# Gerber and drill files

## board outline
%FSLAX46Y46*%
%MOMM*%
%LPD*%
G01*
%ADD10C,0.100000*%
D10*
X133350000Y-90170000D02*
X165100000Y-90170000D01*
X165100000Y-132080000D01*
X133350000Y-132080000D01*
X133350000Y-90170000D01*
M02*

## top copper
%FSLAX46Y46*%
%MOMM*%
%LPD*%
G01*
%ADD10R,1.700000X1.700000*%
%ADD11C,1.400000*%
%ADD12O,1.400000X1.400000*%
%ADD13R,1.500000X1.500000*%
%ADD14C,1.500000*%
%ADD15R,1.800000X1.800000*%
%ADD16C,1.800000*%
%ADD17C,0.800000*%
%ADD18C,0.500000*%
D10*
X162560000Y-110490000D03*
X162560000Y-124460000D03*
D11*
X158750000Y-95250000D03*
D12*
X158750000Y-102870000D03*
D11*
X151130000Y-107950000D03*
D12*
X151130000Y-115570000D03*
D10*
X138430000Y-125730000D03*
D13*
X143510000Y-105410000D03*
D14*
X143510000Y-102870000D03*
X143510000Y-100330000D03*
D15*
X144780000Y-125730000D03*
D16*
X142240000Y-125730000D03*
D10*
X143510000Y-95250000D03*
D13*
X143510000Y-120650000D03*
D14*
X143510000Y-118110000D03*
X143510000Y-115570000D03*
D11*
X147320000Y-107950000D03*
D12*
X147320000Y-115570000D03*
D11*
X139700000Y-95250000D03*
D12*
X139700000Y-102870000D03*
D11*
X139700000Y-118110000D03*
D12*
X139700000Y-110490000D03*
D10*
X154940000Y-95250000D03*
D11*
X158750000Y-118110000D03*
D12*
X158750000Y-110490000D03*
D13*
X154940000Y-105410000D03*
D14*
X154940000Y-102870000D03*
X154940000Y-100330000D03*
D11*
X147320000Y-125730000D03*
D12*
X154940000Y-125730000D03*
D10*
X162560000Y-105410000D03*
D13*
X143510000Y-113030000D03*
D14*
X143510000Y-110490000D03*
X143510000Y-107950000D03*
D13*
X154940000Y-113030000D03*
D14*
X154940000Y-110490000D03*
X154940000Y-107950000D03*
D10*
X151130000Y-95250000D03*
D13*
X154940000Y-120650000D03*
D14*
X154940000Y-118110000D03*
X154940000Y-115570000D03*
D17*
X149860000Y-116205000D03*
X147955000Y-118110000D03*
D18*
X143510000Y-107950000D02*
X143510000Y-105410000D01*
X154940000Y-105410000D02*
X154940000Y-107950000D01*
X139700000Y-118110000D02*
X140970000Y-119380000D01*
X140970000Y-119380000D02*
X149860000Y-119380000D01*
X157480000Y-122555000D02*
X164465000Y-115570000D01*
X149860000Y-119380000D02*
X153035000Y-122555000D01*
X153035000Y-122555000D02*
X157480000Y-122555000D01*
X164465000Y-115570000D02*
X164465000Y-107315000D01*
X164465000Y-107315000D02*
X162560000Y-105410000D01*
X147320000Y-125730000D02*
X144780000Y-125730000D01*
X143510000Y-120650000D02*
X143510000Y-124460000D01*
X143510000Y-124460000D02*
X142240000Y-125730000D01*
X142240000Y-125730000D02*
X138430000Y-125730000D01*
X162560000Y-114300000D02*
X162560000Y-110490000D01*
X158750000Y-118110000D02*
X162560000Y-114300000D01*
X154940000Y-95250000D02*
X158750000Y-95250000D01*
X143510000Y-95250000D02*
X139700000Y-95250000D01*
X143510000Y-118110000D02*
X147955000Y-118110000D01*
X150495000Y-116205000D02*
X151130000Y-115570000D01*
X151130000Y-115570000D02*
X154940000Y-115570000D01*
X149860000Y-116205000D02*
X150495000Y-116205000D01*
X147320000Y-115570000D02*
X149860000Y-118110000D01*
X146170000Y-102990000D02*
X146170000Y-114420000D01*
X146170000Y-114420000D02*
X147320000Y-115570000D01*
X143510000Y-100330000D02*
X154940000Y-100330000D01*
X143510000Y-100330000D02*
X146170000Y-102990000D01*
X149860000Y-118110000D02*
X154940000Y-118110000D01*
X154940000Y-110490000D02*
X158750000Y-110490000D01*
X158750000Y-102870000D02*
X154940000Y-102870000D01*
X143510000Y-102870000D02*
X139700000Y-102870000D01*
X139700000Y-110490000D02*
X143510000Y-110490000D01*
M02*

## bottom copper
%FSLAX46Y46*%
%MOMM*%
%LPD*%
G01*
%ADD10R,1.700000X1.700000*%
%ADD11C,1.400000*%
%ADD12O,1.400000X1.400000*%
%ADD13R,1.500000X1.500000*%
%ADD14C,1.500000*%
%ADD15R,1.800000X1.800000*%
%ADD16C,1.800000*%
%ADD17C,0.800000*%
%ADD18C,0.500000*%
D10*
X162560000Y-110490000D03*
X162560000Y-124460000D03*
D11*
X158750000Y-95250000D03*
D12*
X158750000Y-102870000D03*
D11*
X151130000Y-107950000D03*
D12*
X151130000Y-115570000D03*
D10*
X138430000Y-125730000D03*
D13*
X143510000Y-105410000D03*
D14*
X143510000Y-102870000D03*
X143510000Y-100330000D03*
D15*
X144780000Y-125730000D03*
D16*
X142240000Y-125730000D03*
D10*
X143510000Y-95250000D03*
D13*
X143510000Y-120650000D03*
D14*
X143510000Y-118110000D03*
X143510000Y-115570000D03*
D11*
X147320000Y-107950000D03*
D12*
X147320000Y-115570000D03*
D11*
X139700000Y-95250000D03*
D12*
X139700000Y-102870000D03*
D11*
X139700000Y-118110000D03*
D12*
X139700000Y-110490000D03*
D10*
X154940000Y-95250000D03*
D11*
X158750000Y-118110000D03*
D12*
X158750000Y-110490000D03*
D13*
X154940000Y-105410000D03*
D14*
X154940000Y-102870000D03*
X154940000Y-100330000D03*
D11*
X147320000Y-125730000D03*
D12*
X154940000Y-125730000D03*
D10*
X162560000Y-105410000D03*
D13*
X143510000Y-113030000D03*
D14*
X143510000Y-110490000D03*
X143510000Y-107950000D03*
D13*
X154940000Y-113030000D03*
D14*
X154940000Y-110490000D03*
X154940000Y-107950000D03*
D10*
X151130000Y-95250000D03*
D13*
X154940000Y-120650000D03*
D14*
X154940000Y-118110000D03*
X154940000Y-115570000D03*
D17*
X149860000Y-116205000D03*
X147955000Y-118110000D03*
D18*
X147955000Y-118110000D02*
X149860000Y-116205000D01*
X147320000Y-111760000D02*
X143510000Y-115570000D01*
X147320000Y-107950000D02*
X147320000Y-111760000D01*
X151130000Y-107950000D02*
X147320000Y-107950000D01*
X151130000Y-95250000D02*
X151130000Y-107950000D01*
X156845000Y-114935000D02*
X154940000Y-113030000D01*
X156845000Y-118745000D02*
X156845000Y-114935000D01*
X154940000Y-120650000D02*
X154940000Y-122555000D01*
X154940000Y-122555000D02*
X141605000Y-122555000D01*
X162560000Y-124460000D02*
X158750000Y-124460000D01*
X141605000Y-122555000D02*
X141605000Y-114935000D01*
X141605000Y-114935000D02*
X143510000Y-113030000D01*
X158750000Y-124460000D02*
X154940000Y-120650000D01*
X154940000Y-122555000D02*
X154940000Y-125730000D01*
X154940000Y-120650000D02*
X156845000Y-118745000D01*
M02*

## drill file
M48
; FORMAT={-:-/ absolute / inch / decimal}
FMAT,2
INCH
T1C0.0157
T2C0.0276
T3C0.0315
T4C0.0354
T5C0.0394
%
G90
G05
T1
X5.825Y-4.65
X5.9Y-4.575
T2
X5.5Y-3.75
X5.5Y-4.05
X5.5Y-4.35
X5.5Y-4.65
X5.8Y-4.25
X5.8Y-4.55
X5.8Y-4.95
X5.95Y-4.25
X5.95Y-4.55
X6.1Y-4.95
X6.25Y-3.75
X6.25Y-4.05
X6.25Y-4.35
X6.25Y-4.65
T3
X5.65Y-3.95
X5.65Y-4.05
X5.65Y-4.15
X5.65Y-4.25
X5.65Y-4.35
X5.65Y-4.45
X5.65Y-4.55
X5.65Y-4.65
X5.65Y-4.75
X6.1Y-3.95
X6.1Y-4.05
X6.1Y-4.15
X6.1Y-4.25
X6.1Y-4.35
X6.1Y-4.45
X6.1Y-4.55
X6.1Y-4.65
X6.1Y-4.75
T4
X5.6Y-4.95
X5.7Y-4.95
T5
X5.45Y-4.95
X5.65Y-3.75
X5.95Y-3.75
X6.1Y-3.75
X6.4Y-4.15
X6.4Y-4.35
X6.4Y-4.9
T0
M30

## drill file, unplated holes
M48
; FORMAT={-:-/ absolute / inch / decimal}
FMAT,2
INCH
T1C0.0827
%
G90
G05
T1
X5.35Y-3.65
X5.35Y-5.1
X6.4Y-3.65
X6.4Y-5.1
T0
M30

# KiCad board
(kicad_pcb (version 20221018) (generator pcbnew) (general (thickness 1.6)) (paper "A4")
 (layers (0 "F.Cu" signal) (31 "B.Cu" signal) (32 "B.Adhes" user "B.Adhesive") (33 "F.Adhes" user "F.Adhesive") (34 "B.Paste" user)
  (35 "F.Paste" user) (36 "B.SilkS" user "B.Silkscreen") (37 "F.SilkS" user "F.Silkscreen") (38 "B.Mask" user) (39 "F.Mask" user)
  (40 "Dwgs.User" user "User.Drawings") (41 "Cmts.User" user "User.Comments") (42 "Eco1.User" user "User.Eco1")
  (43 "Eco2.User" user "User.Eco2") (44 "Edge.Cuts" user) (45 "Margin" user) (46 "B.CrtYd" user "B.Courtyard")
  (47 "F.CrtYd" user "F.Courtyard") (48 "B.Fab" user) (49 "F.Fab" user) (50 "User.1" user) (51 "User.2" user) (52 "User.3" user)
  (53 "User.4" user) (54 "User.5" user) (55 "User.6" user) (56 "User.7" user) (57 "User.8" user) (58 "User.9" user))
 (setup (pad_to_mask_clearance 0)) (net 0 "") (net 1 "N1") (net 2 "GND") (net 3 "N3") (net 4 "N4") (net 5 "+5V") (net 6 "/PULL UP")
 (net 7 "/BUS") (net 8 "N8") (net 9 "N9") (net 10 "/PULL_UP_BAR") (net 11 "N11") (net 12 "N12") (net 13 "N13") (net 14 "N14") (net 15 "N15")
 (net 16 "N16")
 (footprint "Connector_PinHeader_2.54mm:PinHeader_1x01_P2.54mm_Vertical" (layer "F.Cu") (at 162.56 110.49)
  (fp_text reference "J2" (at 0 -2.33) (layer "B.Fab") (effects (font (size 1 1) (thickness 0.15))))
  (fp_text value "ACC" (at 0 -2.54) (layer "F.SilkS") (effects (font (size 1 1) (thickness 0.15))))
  (pad "1" thru_hole rect (at 0 0) (size 1.7 1.7) (drill 1) (layers "*.Cu" "*.Mask") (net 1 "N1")))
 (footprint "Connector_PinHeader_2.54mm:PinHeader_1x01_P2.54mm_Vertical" (layer "F.Cu") (at 162.56 124.46)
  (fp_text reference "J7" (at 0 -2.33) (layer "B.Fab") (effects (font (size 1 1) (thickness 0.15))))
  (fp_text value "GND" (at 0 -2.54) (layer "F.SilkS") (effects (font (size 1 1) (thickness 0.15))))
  (pad "1" thru_hole rect (at 0 0) (size 1.7 1.7) (drill 1) (layers "*.Cu" "*.Mask") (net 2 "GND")))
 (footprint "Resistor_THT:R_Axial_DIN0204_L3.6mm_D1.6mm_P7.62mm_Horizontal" (layer "F.Cu") (at 158.75 95.25 -90)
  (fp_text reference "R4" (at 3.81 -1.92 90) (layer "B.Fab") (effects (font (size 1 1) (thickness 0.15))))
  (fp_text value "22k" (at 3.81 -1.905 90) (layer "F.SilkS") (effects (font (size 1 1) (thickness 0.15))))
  (pad "1" thru_hole circle (at 0 0 270) (size 1.4 1.4) (drill 0.7) (layers "*.Cu" "*.Mask") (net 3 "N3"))
  (pad "2" thru_hole oval (at 7.62 0 270) (size 1.4 1.4) (drill 0.7) (layers "*.Cu" "*.Mask") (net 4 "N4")))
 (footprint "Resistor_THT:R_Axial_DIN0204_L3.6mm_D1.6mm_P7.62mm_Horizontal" (layer "F.Cu") (at 151.13 107.95 -90)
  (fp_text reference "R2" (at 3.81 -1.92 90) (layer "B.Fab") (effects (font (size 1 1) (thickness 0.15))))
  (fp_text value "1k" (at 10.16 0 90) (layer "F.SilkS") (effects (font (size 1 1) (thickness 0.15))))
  (pad "1" thru_hole circle (at 0 0 270) (size 1.4 1.4) (drill 0.7) (layers "*.Cu" "*.Mask") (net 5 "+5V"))
  (pad "2" thru_hole oval (at 7.62 0 270) (size 1.4 1.4) (drill 0.7) (layers "*.Cu" "*.Mask") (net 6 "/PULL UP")))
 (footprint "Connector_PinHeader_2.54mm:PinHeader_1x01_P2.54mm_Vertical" (layer "F.Cu") (at 138.43 125.73)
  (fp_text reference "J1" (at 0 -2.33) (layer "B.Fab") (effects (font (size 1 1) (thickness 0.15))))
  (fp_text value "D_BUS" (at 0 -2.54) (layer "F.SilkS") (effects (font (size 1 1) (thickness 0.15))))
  (pad "1" thru_hole rect (at 0 0) (size 1.7 1.7) (drill 1) (layers "*.Cu" "*.Mask") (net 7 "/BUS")))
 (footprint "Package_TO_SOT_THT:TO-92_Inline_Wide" (layer "F.Cu") (at 143.51 105.41 90)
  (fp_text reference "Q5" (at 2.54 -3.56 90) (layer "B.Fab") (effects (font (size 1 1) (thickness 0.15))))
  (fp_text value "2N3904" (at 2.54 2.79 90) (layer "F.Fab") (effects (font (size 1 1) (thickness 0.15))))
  (pad "1" thru_hole rect (at 0 0 90) (size 1.5 1.5) (drill 0.8) (layers "*.Cu" "*.Mask") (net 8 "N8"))
  (pad "2" thru_hole circle (at 2.54 0 90) (size 1.5 1.5) (drill 0.8) (layers "*.Cu" "*.Mask") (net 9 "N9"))
  (pad "3" thru_hole circle (at 5.08 0 90) (size 1.5 1.5) (drill 0.8) (layers "*.Cu" "*.Mask") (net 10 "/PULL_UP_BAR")))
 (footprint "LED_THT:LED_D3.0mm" (layer "F.Cu") (at 144.78 125.73 180)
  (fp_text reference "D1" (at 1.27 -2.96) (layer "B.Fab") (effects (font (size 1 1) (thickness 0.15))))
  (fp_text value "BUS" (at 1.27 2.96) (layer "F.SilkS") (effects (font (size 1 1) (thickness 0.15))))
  (pad "1" thru_hole rect (at 0 0 180) (size 1.8 1.8) (drill 0.9) (layers "*.Cu" "*.Mask") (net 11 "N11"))
  (pad "2" thru_hole circle (at 2.54 0 180) (size 1.8 1.8) (drill 0.9) (layers "*.Cu" "*.Mask") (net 7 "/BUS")))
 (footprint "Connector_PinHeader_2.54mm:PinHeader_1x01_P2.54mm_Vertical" (layer "F.Cu") (at 143.51 95.25)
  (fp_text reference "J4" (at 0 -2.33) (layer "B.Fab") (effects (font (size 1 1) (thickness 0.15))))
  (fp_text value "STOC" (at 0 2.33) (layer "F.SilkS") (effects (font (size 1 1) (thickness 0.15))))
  (pad "1" thru_hole rect (at 0 0) (size 1.7 1.7) (drill 1) (layers "*.Cu" "*.Mask") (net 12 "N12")))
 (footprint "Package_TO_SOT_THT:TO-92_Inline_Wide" (layer "F.Cu") (at 143.51 120.65 90)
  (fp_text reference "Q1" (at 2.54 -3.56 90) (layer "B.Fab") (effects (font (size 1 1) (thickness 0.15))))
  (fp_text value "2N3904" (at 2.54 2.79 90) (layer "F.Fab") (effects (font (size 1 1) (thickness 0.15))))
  (pad "1" thru_hole rect (at 0 0 90) (size 1.5 1.5) (drill 0.8) (layers "*.Cu" "*.Mask") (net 7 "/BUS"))
  (pad "2" thru_hole circle (at 2.54 0 90) (size 1.5 1.5) (drill 0.8) (layers "*.Cu" "*.Mask") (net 6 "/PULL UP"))
  (pad "3" thru_hole circle (at 5.08 0 90) (size 1.5 1.5) (drill 0.8) (layers "*.Cu" "*.Mask") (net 5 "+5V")))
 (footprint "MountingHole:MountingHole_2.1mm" (layer "F.Cu") (at 135.89 92.71)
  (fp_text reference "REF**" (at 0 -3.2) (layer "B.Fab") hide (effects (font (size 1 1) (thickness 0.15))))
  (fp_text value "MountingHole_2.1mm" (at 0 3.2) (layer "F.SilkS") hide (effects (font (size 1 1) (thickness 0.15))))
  (pad "" np_thru_hole circle (at 0 0) (size 2.1 2.1) (drill 2.1) (layers "F&B.Cu" "*.Mask")))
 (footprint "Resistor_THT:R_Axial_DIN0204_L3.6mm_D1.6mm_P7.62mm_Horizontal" (layer "F.Cu") (at 147.32 107.95 -90)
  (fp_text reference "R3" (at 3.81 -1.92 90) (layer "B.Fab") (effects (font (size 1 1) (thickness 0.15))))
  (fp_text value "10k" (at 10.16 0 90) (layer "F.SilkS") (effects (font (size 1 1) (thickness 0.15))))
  (pad "1" thru_hole circle (at 0 0 270) (size 1.4 1.4) (drill 0.7) (layers "*.Cu" "*.Mask") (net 5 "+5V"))
  (pad "2" thru_hole oval (at 7.62 0 270) (size 1.4 1.4) (drill 0.7) (layers "*.Cu" "*.Mask") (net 10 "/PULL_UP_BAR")))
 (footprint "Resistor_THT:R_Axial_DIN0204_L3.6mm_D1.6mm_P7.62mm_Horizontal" (layer "F.Cu") (at 139.7 95.25 -90)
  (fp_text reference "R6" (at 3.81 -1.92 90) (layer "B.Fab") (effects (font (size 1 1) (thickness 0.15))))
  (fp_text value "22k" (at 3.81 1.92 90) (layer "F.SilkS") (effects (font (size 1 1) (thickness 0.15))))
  (pad "1" thru_hole circle (at 0 0 270) (size 1.4 1.4) (drill 0.7) (layers "*.Cu" "*.Mask") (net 12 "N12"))
  (pad "2" thru_hole oval (at 7.62 0 270) (size 1.4 1.4) (drill 0.7) (layers "*.Cu" "*.Mask") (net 9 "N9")))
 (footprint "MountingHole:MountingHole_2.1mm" (layer "F.Cu") (at 135.89 129.54)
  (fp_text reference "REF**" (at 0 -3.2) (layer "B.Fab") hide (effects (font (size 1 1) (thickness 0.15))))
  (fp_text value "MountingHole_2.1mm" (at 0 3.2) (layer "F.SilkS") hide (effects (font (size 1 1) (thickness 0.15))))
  (pad "" np_thru_hole circle (at 0 0) (size 2.1 2.1) (drill 2.1) (layers "F&B.Cu" "*.Mask")))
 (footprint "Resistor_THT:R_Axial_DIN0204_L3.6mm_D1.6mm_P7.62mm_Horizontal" (layer "F.Cu") (at 139.7 118.11 90)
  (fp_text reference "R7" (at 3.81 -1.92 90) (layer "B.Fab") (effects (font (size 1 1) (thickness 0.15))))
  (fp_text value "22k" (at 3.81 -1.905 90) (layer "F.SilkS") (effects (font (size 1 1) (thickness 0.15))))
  (pad "1" thru_hole circle (at 0 0 90) (size 1.4 1.4) (drill 0.7) (layers "*.Cu" "*.Mask") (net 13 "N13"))
  (pad "2" thru_hole oval (at 7.62 0 90) (size 1.4 1.4) (drill 0.7) (layers "*.Cu" "*.Mask") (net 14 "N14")))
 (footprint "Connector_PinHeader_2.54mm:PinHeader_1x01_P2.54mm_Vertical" (layer "F.Cu") (at 154.94 95.25)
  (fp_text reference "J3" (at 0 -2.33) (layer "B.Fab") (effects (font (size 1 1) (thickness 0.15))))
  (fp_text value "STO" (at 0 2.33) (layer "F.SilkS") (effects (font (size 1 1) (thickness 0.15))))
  (pad "1" thru_hole rect (at 0 0) (size 1.7 1.7) (drill 1) (layers "*.Cu" "*.Mask") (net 3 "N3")))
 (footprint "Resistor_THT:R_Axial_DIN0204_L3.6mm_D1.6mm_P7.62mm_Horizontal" (layer "F.Cu") (at 158.75 118.11 90)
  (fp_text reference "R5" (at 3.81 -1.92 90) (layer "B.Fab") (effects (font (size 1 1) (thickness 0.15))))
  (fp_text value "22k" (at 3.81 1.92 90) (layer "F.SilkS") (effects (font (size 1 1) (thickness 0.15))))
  (pad "1" thru_hole circle (at 0 0 90) (size 1.4 1.4) (drill 0.7) (layers "*.Cu" "*.Mask") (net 1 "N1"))
  (pad "2" thru_hole oval (at 7.62 0 90) (size 1.4 1.4) (drill 0.7) (layers "*.Cu" "*.Mask") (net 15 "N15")))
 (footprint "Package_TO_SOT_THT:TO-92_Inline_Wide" (layer "F.Cu") (at 154.94 105.41 90)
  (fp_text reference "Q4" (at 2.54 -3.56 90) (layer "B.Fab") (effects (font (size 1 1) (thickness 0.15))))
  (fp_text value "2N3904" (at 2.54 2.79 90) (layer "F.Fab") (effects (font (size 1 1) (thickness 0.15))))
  (pad "1" thru_hole rect (at 0 0 90) (size 1.5 1.5) (drill 0.8) (layers "*.Cu" "*.Mask") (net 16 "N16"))
  (pad "2" thru_hole circle (at 2.54 0 90) (size 1.5 1.5) (drill 0.8) (layers "*.Cu" "*.Mask") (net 4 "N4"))
  (pad "3" thru_hole circle (at 5.08 0 90) (size 1.5 1.5) (drill 0.8) (layers "*.Cu" "*.Mask") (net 10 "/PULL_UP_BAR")))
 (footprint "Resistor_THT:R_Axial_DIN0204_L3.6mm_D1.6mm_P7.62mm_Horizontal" (layer "F.Cu") (at 147.32 125.73)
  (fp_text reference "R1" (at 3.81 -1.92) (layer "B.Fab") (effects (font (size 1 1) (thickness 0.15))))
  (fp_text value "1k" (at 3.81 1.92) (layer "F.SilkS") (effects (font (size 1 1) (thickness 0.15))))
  (pad "1" thru_hole circle (at 0 0) (size 1.4 1.4) (drill 0.7) (layers "*.Cu" "*.Mask") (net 11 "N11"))
  (pad "2" thru_hole oval (at 7.62 0) (size 1.4 1.4) (drill 0.7) (layers "*.Cu" "*.Mask") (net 2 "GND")))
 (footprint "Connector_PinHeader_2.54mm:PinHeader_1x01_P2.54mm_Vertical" (layer "F.Cu") (at 162.56 105.41)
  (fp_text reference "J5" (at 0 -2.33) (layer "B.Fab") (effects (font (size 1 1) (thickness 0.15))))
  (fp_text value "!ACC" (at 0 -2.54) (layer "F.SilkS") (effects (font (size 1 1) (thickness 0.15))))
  (pad "1" thru_hole rect (at 0 0) (size 1.7 1.7) (drill 1) (layers "*.Cu" "*.Mask") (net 13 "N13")))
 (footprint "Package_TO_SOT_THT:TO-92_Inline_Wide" (layer "F.Cu") (at 143.51 113.03 90)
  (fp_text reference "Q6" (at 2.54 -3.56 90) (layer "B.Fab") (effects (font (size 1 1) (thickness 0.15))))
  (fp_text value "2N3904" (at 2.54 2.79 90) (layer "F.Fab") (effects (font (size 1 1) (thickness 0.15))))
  (pad "1" thru_hole rect (at 0 0 90) (size 1.5 1.5) (drill 0.8) (layers "*.Cu" "*.Mask") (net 2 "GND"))
  (pad "2" thru_hole circle (at 2.54 0 90) (size 1.5 1.5) (drill 0.8) (layers "*.Cu" "*.Mask") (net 14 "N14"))
  (pad "3" thru_hole circle (at 5.08 0 90) (size 1.5 1.5) (drill 0.8) (layers "*.Cu" "*.Mask") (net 8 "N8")))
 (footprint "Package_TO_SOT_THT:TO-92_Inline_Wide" (layer "F.Cu") (at 154.94 113.03 90)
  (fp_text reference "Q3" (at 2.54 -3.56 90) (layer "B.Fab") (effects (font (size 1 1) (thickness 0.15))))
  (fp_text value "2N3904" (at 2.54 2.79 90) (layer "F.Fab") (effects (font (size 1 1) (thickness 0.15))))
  (pad "1" thru_hole rect (at 0 0 90) (size 1.5 1.5) (drill 0.8) (layers "*.Cu" "*.Mask") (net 2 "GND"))
  (pad "2" thru_hole circle (at 2.54 0 90) (size 1.5 1.5) (drill 0.8) (layers "*.Cu" "*.Mask") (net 15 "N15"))
  (pad "3" thru_hole circle (at 5.08 0 90) (size 1.5 1.5) (drill 0.8) (layers "*.Cu" "*.Mask") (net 16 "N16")))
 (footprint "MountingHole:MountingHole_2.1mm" (layer "F.Cu") (at 162.56 129.54)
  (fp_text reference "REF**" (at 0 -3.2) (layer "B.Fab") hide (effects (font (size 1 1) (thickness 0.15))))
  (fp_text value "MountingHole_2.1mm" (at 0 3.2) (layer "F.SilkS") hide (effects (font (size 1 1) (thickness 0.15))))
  (pad "" np_thru_hole circle (at 0 0) (size 2.1 2.1) (drill 2.1) (layers "*.Cu" "*.Mask")))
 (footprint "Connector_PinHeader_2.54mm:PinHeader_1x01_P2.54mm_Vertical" (layer "F.Cu") (at 151.13 95.25)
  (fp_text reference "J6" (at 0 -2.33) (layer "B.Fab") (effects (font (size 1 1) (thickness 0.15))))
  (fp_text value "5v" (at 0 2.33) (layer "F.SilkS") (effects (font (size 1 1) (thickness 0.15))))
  (pad "1" thru_hole rect (at 0 0) (size 1.7 1.7) (drill 1) (layers "*.Cu" "*.Mask") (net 5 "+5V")))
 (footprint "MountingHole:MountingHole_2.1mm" (layer "F.Cu") (at 162.56 92.71)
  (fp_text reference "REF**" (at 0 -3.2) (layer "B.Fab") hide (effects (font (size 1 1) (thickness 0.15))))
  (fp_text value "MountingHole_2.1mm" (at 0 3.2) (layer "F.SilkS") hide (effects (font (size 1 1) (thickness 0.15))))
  (pad "" np_thru_hole circle (at 0 0) (size 2.1 2.1) (drill 2.1) (layers "F&B.Cu" "*.Mask")))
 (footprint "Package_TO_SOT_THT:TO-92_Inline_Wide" (layer "F.Cu") (at 154.94 120.65 90)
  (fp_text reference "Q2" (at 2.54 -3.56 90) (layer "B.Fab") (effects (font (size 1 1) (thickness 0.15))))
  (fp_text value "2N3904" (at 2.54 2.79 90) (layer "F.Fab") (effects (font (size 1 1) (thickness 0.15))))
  (pad "1" thru_hole rect (at 0 0 90) (size 1.5 1.5) (drill 0.8) (layers "*.Cu" "*.Mask") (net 2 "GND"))
  (pad "2" thru_hole circle (at 2.54 0 90) (size 1.5 1.5) (drill 0.8) (layers "*.Cu" "*.Mask") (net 10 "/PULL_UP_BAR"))
  (pad "3" thru_hole circle (at 5.08 0 90) (size 1.5 1.5) (drill 0.8) (layers "*.Cu" "*.Mask") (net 6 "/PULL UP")))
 (gr_rect (start 133.35 90.17) (end 165.1 132.08) (stroke (width 0.1) (type default)) (fill none) (layer "Edge.Cuts"))
 (segment (start 147.32 125.73) (end 144.78 125.73) (width 0.5) (layer "F.Cu") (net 11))
 (segment (start 143.51 120.65) (end 143.51 124.46) (width 0.5) (layer "F.Cu") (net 7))
 (segment (start 143.51 124.46) (end 142.24 125.73) (width 0.5) (layer "F.Cu") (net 7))
 (segment (start 142.24 125.73) (end 138.43 125.73) (width 0.5) (layer "F.Cu") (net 7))
 (segment (start 162.56 114.3) (end 162.56 110.49) (width 0.5) (layer "F.Cu") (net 1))
 (segment (start 158.75 118.11) (end 162.56 114.3) (width 0.5) (layer "F.Cu") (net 1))
 (segment (start 154.94 95.25) (end 158.75 95.25) (width 0.5) (layer "F.Cu") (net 3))
 (segment (start 143.51 95.25) (end 139.7 95.25) (width 0.5) (layer "F.Cu") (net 12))
 (segment (start 164.465 107.315) (end 162.56 105.41) (width 0.5) (layer "F.Cu") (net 13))
 (segment (start 157.48 122.555) (end 164.465 115.57) (width 0.5) (layer "F.Cu") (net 13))
 (segment (start 149.86 119.38) (end 153.035 122.555) (width 0.5) (layer "F.Cu") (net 13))
 (segment (start 139.7 118.11) (end 140.97 119.38) (width 0.5) (layer "F.Cu") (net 13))
 (segment (start 164.465 115.57) (end 164.465 107.315) (width 0.5) (layer "F.Cu") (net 13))
 (segment (start 153.035 122.555) (end 157.48 122.555) (width 0.5) (layer "F.Cu") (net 13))
 (segment (start 140.97 119.38) (end 149.86 119.38) (width 0.5) (layer "F.Cu") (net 13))
 (segment (start 143.51 118.11) (end 147.955 118.11) (width 0.5) (layer "F.Cu") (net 6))
 (segment (start 150.495 116.205) (end 151.13 115.57) (width 0.5) (layer "F.Cu") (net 6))
 (segment (start 151.13 115.57) (end 154.94 115.57) (width 0.5) (layer "F.Cu") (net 6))
 (segment (start 149.86 116.205) (end 150.495 116.205) (width 0.5) (layer "F.Cu") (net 6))
 (via (at 149.86 116.205) (size 0.8) (drill 0.4) (layers "F.Cu" "B.Cu") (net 6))
 (via (at 147.955 118.11) (size 0.8) (drill 0.4) (layers "F.Cu" "B.Cu") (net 6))
 (segment (start 147.955 118.11) (end 149.86 116.205) (width 0.5) (layer "B.Cu") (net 6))
 (segment (start 147.32 111.76) (end 143.51 115.57) (width 0.5) (layer "B.Cu") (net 5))
 (segment (start 147.32 107.95) (end 147.32 111.76) (width 0.5) (layer "B.Cu") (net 5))
 (segment (start 151.13 107.95) (end 147.32 107.95) (width 0.5) (layer "B.Cu") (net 5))
 (segment (start 151.13 95.25) (end 151.13 107.95) (width 0.5) (layer "B.Cu") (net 5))
 (segment (start 156.845 114.935) (end 154.94 113.03) (width 0.5) (layer "B.Cu") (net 2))
 (segment (start 156.845 118.745) (end 156.845 114.935) (width 0.5) (layer "B.Cu") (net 2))
 (segment (start 154.94 120.65) (end 154.94 122.555) (width 0.5) (layer "B.Cu") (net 2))
 (segment (start 154.94 122.555) (end 141.605 122.555) (width 0.5) (layer "B.Cu") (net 2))
 (segment (start 162.56 124.46) (end 158.75 124.46) (width 0.5) (layer "B.Cu") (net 2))
 (segment (start 141.605 122.555) (end 141.605 114.935) (width 0.5) (layer "B.Cu") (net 2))
 (segment (start 141.605 114.935) (end 143.51 113.03) (width 0.5) (layer "B.Cu") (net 2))
 (segment (start 158.75 124.46) (end 154.94 120.65) (width 0.5) (layer "B.Cu") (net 2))
 (segment (start 154.94 122.555) (end 154.94 125.73) (width 0.5) (layer "B.Cu") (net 2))
 (segment (start 154.94 120.65) (end 156.845 118.745) (width 0.5) (layer "B.Cu") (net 2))
 (segment (start 147.32 115.57) (end 149.86 118.11) (width 0.5) (layer "F.Cu") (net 10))
 (segment (start 146.17 102.99) (end 146.17 114.42) (width 0.5) (layer "F.Cu") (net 10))
 (segment (start 146.17 114.42) (end 147.32 115.57) (width 0.5) (layer "F.Cu") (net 10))
 (segment (start 143.51 100.33) (end 154.94 100.33) (width 0.5) (layer "F.Cu") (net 10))
 (segment (start 143.51 100.33) (end 146.17 102.99) (width 0.5) (layer "F.Cu") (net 10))
 (segment (start 149.86 118.11) (end 154.94 118.11) (width 0.5) (layer "F.Cu") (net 10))
 (segment (start 154.94 110.49) (end 158.75 110.49) (width 0.5) (layer "F.Cu") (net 15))
 (segment (start 154.94 105.41) (end 154.94 107.95) (width 0.5) (layer "F.Cu") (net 16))
 (segment (start 158.75 102.87) (end 154.94 102.87) (width 0.5) (layer "F.Cu") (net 4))
 (segment (start 143.51 107.95) (end 143.51 105.41) (width 0.5) (layer "F.Cu") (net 8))
 (segment (start 143.51 102.87) (end 139.7 102.87) (width 0.5) (layer "F.Cu") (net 9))
 (segment (start 139.7 110.49) (end 143.51 110.49) (width 0.5) (layer "F.Cu") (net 14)))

